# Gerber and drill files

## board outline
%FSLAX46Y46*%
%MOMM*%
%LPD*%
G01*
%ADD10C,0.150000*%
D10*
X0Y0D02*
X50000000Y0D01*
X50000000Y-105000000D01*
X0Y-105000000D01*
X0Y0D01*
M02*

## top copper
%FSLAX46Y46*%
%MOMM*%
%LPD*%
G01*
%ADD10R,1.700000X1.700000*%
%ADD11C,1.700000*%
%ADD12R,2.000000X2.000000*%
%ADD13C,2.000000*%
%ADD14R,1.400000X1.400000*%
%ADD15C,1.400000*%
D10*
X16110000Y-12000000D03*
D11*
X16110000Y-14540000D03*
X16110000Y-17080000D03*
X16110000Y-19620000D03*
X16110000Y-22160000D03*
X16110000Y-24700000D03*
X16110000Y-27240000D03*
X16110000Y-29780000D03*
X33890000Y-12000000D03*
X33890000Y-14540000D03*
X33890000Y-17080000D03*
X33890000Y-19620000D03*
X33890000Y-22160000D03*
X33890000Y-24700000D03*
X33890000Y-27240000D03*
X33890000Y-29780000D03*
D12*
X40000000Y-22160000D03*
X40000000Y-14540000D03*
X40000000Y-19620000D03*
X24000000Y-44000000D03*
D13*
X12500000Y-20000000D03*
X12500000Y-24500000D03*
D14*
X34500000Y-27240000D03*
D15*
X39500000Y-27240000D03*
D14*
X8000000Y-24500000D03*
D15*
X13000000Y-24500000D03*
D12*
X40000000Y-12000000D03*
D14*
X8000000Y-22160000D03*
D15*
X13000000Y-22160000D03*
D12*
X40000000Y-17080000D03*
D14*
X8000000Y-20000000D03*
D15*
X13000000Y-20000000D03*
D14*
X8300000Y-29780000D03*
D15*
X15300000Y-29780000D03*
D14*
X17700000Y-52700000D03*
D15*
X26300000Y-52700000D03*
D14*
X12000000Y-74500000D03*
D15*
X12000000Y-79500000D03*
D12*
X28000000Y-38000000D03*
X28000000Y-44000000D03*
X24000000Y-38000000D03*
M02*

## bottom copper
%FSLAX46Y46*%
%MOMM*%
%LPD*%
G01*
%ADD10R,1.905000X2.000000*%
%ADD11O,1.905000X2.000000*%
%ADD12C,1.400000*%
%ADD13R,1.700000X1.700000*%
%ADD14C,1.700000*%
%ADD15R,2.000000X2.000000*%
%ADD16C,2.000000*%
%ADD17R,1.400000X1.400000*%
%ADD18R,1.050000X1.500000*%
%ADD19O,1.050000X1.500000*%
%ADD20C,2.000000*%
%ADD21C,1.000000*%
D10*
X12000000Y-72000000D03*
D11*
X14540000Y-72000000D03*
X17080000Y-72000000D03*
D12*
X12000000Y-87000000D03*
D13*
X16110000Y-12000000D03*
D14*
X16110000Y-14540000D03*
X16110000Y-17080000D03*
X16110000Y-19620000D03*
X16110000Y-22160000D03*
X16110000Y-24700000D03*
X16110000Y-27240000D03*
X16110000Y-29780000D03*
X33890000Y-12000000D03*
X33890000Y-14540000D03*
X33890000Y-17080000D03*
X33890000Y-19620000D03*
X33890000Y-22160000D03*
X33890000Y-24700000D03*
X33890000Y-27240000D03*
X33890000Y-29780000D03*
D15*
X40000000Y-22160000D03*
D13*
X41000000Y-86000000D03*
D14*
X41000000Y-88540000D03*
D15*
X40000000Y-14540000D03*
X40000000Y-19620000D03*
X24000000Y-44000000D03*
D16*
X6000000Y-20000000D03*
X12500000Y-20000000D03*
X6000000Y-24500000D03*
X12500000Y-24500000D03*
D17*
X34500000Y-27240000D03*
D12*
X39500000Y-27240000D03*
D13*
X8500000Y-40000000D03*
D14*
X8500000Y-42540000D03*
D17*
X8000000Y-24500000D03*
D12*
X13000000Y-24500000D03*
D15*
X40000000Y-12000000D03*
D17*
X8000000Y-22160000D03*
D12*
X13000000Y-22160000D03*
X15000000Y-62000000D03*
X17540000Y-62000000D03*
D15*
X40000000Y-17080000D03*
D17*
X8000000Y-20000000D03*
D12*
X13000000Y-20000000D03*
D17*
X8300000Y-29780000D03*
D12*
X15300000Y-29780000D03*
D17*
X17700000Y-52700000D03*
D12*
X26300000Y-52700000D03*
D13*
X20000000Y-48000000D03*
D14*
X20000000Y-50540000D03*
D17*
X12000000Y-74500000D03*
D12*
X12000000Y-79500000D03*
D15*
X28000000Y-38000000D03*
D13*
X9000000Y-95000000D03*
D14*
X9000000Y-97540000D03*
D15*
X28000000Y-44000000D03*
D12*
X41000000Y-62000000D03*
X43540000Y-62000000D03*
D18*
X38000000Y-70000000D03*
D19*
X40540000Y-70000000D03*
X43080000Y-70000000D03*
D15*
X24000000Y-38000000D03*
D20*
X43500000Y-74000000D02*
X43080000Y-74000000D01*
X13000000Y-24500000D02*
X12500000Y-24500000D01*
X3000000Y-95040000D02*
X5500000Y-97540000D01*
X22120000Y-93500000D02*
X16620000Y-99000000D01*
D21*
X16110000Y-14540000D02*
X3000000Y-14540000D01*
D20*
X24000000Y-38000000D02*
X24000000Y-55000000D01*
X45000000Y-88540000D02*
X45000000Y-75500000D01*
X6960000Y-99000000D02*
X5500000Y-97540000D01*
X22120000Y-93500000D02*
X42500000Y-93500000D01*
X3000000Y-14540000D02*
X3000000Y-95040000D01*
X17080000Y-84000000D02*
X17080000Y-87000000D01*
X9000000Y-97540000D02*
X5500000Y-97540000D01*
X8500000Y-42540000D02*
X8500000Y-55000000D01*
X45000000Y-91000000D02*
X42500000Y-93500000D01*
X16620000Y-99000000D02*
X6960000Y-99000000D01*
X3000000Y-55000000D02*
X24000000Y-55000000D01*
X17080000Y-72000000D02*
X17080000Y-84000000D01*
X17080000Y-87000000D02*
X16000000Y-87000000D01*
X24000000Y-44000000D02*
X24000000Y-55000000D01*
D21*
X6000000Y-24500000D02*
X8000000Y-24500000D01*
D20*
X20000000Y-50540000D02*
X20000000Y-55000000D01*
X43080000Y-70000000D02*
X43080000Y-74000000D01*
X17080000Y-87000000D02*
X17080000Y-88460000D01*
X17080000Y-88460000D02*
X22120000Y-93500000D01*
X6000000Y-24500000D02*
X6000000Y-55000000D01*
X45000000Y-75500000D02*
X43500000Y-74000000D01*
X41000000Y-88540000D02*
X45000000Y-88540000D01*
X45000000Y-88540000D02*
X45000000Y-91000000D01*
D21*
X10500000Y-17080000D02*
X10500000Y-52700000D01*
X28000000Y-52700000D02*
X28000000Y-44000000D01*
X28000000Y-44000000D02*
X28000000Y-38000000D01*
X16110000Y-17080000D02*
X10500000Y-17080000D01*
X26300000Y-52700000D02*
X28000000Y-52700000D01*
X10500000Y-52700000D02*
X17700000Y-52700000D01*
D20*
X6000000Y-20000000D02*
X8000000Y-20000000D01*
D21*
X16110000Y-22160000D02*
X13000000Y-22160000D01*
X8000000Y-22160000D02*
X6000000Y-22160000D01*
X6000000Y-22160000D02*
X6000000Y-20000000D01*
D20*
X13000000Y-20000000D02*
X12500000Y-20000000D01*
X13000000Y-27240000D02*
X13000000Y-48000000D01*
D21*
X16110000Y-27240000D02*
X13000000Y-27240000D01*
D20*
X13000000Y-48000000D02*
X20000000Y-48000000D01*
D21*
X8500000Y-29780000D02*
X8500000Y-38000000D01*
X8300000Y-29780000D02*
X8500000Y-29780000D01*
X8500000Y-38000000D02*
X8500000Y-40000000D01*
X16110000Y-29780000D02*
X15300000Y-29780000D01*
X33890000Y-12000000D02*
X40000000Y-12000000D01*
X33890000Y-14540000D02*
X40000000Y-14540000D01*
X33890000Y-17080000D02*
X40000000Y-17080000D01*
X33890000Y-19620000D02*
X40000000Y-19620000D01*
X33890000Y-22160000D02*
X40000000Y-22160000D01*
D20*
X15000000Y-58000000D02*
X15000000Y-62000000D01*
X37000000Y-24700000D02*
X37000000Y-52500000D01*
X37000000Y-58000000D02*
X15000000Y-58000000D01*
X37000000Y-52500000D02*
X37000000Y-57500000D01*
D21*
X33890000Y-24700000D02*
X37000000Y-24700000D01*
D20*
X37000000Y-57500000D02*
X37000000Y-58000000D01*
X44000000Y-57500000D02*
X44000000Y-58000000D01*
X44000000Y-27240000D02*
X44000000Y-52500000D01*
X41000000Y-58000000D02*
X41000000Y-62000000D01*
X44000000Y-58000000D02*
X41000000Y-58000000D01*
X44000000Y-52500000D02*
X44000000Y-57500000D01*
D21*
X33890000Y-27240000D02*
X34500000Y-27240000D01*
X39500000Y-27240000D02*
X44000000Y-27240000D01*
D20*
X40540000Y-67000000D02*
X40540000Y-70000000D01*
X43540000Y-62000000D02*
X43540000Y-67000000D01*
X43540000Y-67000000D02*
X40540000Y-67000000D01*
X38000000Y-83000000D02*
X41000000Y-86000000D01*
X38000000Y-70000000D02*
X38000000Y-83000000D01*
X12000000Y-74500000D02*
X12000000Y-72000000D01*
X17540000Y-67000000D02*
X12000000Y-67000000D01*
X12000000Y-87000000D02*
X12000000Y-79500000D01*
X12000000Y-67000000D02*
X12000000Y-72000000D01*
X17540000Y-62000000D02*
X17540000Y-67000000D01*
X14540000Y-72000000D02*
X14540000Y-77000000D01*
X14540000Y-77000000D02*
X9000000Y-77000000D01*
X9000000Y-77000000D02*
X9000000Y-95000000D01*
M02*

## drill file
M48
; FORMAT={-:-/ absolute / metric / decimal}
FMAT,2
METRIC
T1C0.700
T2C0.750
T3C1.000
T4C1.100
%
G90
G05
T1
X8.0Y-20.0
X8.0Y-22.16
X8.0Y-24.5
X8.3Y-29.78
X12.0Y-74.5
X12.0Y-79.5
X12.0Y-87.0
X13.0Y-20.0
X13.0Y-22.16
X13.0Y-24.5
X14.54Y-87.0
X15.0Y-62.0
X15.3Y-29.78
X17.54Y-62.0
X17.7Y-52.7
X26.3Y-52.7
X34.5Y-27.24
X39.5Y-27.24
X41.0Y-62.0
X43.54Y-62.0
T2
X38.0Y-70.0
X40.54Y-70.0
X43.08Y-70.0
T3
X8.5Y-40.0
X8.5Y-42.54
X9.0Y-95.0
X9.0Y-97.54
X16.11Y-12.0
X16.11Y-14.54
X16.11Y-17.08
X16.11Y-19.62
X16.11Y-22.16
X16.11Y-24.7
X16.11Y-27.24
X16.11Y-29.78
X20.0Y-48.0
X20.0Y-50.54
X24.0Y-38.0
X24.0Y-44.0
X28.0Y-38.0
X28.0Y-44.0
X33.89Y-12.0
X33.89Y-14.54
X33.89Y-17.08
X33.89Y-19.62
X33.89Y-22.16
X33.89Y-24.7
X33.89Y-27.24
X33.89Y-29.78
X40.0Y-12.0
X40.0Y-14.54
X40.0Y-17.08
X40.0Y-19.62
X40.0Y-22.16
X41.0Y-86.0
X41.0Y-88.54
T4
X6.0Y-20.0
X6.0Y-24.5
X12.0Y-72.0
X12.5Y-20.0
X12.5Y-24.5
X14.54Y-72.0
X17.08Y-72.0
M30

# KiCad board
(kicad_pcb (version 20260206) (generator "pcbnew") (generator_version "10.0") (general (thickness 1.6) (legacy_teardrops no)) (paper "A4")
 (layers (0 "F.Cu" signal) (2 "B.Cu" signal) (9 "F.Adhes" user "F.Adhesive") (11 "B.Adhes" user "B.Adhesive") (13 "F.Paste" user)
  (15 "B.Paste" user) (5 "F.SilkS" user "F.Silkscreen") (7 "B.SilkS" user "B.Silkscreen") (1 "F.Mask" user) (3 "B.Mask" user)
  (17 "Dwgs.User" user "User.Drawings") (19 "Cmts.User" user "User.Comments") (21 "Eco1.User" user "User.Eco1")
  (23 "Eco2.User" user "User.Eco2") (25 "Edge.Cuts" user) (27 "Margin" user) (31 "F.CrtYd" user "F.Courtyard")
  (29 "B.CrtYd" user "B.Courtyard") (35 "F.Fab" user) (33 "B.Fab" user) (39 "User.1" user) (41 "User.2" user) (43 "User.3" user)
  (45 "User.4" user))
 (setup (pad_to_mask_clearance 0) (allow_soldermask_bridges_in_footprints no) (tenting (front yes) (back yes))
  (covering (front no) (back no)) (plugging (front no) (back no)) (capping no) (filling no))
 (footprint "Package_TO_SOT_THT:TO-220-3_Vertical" (layer "F.Cu") (at 12 72)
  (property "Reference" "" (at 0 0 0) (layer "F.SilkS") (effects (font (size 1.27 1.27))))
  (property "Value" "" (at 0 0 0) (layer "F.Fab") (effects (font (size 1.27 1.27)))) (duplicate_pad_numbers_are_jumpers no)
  (pad "1" thru_hole rect (at 0 0) (size 1.905 2) (drill 1.1) (layers "*.Cu" "*.Mask") (remove_unused_layers yes) (keep_end_layers no)
   (zone_layer_connections) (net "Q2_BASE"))
  (pad "2" thru_hole oval (at 2.54 0) (size 1.905 2) (drill 1.1) (layers "*.Cu" "*.Mask") (remove_unused_layers yes) (keep_end_layers no)
   (zone_layer_connections) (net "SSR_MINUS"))
  (pad "3" thru_hole oval (at 5.08 0) (size 1.905 2) (drill 1.1) (layers "*.Cu" "*.Mask") (remove_unused_layers yes) (keep_end_layers no)
   (zone_layer_connections) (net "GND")))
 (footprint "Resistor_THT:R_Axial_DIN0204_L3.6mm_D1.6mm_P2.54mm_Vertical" (layer "F.Cu") (at 12 87)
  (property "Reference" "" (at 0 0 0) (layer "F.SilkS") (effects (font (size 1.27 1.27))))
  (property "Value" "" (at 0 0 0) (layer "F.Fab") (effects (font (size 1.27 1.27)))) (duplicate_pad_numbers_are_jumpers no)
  (pad "1" thru_hole circle (at 0 0) (size 1.4 1.4) (drill 0.7) (layers "*.Cu" "*.Mask") (remove_unused_layers yes) (keep_end_layers no)
   (zone_layer_connections) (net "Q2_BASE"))
  (pad "2" thru_hole circle (at 2.54 0) (size 1.4 1.4) (drill 0.7) (layers "*.Cu" "*.Mask") (remove_unused_layers yes) (keep_end_layers no)
   (zone_layer_connections) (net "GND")))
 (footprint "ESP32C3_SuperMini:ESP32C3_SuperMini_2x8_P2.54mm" (layer "F.Cu") (at 16.11 12)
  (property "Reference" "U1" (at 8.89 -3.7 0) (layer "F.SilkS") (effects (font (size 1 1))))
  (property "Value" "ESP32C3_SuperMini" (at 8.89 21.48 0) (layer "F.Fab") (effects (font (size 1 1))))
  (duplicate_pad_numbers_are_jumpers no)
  (pad "1" thru_hole rect (at 0 0) (size 1.7 1.7) (drill 1) (layers "*.Cu" "*.Mask") (remove_unused_layers no))
  (pad "2" thru_hole circle (at 0 2.54) (size 1.7 1.7) (drill 1) (layers "*.Cu" "*.Mask") (remove_unused_layers no) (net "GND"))
  (pad "3" thru_hole circle (at 0 5.08) (size 1.7 1.7) (drill 1) (layers "*.Cu" "*.Mask") (remove_unused_layers no) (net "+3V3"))
  (pad "4" thru_hole circle (at 0 7.62) (size 1.7 1.7) (drill 1) (layers "*.Cu" "*.Mask") (remove_unused_layers no))
  (pad "5" thru_hole circle (at 0 10.16) (size 1.7 1.7) (drill 1) (layers "*.Cu" "*.Mask") (remove_unused_layers no) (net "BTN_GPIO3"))
  (pad "6" thru_hole circle (at 0 12.7) (size 1.7 1.7) (drill 1) (layers "*.Cu" "*.Mask") (remove_unused_layers no))
  (pad "7" thru_hole circle (at 0 15.24) (size 1.7 1.7) (drill 1) (layers "*.Cu" "*.Mask") (remove_unused_layers no) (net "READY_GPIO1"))
  (pad "8" thru_hole circle (at 0 17.78) (size 1.7 1.7) (drill 1) (layers "*.Cu" "*.Mask") (remove_unused_layers no) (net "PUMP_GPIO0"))
  (pad "9" thru_hole circle (at 17.78 0) (size 1.7 1.7) (drill 1) (layers "*.Cu" "*.Mask") (remove_unused_layers no) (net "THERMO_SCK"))
  (pad "10" thru_hole circle (at 17.78 2.54) (size 1.7 1.7) (drill 1) (layers "*.Cu" "*.Mask") (remove_unused_layers no) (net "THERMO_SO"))
  (pad "11" thru_hole circle (at 17.78 5.08) (size 1.7 1.7) (drill 1) (layers "*.Cu" "*.Mask") (remove_unused_layers no) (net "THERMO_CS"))
  (pad "12" thru_hole circle (at 17.78 7.62) (size 1.7 1.7) (drill 1) (layers "*.Cu" "*.Mask") (remove_unused_layers no) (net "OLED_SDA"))
  (pad "13" thru_hole circle (at 17.78 10.16) (size 1.7 1.7) (drill 1) (layers "*.Cu" "*.Mask") (remove_unused_layers no) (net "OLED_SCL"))
  (pad "14" thru_hole circle (at 17.78 12.7) (size 1.7 1.7) (drill 1) (layers "*.Cu" "*.Mask") (remove_unused_layers no)
   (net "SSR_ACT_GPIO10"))
  (pad "15" thru_hole circle (at 17.78 15.24) (size 1.7 1.7) (drill 1) (layers "*.Cu" "*.Mask") (remove_unused_layers no)
   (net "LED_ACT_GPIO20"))
  (pad "16" thru_hole circle (at 17.78 17.78) (size 1.7 1.7) (drill 1) (layers "*.Cu" "*.Mask") (remove_unused_layers no)))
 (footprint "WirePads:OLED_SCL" (layer "F.Cu") (at 40 22.16)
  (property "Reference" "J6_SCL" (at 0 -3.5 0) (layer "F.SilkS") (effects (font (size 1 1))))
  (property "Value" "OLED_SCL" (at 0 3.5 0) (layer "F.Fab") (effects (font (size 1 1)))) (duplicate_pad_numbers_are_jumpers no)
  (pad "1" thru_hole rect (at 0 0) (size 2 2) (drill 1) (layers "*.Cu" "*.Mask") (remove_unused_layers no) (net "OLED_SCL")))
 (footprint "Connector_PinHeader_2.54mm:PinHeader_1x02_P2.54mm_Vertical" (layer "F.Cu") (at 41 86)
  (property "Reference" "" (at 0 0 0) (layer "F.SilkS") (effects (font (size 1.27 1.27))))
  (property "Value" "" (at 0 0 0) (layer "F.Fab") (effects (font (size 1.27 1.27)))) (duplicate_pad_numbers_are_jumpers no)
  (pad "1" thru_hole rect (at 0 0) (size 1.7 1.7) (drill 1) (layers "*.Cu" "*.Mask") (remove_unused_layers yes) (keep_end_layers no)
   (zone_layer_connections) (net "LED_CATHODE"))
  (pad "2" thru_hole circle (at 0 2.54) (size 1.7 1.7) (drill 1) (layers "*.Cu" "*.Mask") (remove_unused_layers yes) (keep_end_layers no)
   (zone_layer_connections) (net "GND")))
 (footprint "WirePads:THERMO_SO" (layer "F.Cu") (at 40 14.54)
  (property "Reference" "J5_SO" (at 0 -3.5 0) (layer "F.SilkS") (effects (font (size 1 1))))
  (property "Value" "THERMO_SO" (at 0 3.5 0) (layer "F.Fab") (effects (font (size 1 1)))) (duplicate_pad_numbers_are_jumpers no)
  (pad "1" thru_hole rect (at 0 0) (size 2 2) (drill 1) (layers "*.Cu" "*.Mask") (remove_unused_layers no) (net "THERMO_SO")))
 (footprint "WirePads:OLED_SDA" (layer "F.Cu") (at 40 19.62)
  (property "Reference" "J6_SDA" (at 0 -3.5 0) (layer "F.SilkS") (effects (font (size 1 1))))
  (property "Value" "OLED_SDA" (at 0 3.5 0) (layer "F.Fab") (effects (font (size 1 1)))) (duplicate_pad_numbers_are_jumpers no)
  (pad "1" thru_hole rect (at 0 0) (size 2 2) (drill 1) (layers "*.Cu" "*.Mask") (remove_unused_layers no) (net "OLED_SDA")))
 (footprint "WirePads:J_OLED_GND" (layer "F.Cu") (at 24 44)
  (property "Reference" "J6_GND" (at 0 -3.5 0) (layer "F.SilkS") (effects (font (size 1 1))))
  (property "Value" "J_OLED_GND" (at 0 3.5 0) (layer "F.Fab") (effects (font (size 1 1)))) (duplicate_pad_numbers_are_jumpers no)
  (pad "1" thru_hole rect (at 0 0) (size 2 2) (drill 1) (layers "*.Cu" "*.Mask") (remove_unused_layers no) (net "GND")))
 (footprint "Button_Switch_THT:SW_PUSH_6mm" (layer "F.Cu") (at 6 20)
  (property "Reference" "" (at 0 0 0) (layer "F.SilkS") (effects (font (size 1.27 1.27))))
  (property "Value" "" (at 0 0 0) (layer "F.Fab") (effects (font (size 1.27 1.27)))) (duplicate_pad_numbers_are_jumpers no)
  (pad "1" thru_hole circle (at 0 0 90) (size 2 2) (drill 1.1) (layers "*.Cu" "*.Mask") (remove_unused_layers yes) (keep_end_layers no)
   (zone_layer_connections) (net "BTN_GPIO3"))
  (pad "1" thru_hole circle (at 6.5 0 90) (size 2 2) (drill 1.1) (layers "*.Cu" "*.Mask") (remove_unused_layers yes) (keep_end_layers no)
   (zone_layer_connections) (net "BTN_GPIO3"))
  (pad "2" thru_hole circle (at 0 4.5 90) (size 2 2) (drill 1.1) (layers "*.Cu" "*.Mask") (remove_unused_layers yes) (keep_end_layers no)
   (zone_layer_connections) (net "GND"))
  (pad "2" thru_hole circle (at 6.5 4.5 90) (size 2 2) (drill 1.1) (layers "*.Cu" "*.Mask") (remove_unused_layers yes) (keep_end_layers no)
   (zone_layer_connections) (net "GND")))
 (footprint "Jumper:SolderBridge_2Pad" (layer "F.Cu") (at 34.5 27.24)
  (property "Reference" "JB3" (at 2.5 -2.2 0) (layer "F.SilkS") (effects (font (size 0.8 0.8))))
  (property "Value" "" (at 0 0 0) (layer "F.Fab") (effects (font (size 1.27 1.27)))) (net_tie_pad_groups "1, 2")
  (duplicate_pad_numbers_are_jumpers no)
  (pad "1" thru_hole rect (at 0 0) (size 1.4 1.4) (drill 0.7) (layers "*.Cu" "*.Mask") (remove_unused_layers no) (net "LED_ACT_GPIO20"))
  (pad "2" thru_hole circle (at 5 0) (size 1.4 1.4) (drill 0.7) (layers "*.Cu" "*.Mask") (remove_unused_layers no) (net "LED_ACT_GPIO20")))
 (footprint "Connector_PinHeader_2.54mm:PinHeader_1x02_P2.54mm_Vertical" (layer "F.Cu") (at 8.5 40)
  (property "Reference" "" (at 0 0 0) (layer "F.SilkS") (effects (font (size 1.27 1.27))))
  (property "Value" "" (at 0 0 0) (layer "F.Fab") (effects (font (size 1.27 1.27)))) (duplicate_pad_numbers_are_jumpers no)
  (pad "1" thru_hole rect (at 0 0) (size 1.7 1.7) (drill 1) (layers "*.Cu" "*.Mask") (remove_unused_layers yes) (keep_end_layers no)
   (zone_layer_connections) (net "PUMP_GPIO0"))
  (pad "2" thru_hole circle (at 0 2.54) (size 1.7 1.7) (drill 1) (layers "*.Cu" "*.Mask") (remove_unused_layers yes) (keep_end_layers no)
   (zone_layer_connections) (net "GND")))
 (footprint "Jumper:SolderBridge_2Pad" (layer "F.Cu") (at 8 24.5)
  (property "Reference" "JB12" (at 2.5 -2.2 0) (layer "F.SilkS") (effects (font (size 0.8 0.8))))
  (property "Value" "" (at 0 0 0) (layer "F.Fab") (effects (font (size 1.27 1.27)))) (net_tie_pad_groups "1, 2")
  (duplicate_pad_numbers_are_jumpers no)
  (pad "1" thru_hole rect (at 0 0) (size 1.4 1.4) (drill 0.7) (layers "*.Cu" "*.Mask") (remove_unused_layers no) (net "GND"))
  (pad "2" thru_hole circle (at 5 0) (size 1.4 1.4) (drill 0.7) (layers "*.Cu" "*.Mask") (remove_unused_layers no) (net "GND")))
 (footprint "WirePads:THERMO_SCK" (layer "F.Cu") (at 40 12)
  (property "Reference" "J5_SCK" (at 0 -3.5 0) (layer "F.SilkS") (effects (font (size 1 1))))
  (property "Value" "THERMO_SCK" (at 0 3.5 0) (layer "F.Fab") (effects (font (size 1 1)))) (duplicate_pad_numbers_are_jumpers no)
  (pad "1" thru_hole rect (at 0 0) (size 2 2) (drill 1) (layers "*.Cu" "*.Mask") (remove_unused_layers no) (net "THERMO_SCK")))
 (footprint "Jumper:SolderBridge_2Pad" (layer "F.Cu") (at 8 22.16)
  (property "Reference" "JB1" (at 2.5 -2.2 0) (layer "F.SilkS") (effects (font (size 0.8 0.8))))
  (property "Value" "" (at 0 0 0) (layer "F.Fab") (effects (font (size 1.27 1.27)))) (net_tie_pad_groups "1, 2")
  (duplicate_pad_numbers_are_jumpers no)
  (pad "1" thru_hole rect (at 0 0) (size 1.4 1.4) (drill 0.7) (layers "*.Cu" "*.Mask") (remove_unused_layers no) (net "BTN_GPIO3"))
  (pad "2" thru_hole circle (at 5 0) (size 1.4 1.4) (drill 0.7) (layers "*.Cu" "*.Mask") (remove_unused_layers no) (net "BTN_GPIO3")))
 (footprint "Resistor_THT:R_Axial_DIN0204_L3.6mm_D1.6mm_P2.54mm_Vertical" (layer "F.Cu") (at 15 62)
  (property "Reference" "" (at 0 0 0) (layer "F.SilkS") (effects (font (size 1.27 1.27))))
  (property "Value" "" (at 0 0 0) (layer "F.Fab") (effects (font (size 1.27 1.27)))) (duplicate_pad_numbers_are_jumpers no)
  (pad "1" thru_hole circle (at 0 0) (size 1.4 1.4) (drill 0.7) (layers "*.Cu" "*.Mask") (remove_unused_layers yes) (keep_end_layers no)
   (zone_layer_connections) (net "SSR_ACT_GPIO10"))
  (pad "2" thru_hole circle (at 2.54 0) (size 1.4 1.4) (drill 0.7) (layers "*.Cu" "*.Mask") (remove_unused_layers yes) (keep_end_layers no)
   (zone_layer_connections) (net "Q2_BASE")))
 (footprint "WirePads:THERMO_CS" (layer "F.Cu") (at 40 17.08)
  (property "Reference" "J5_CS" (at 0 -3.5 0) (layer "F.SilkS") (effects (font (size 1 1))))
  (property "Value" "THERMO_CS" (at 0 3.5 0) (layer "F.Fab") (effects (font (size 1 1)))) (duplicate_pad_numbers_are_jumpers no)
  (pad "1" thru_hole rect (at 0 0) (size 2 2) (drill 1) (layers "*.Cu" "*.Mask") (remove_unused_layers no) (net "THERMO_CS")))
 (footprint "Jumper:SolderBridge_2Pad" (layer "F.Cu") (at 8 20)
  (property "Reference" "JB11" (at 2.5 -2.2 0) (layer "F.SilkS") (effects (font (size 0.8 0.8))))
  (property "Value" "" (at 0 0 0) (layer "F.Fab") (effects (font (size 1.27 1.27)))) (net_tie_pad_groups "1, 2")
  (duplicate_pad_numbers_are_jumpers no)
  (pad "1" thru_hole rect (at 0 0) (size 1.4 1.4) (drill 0.7) (layers "*.Cu" "*.Mask") (remove_unused_layers no) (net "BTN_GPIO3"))
  (pad "2" thru_hole circle (at 5 0) (size 1.4 1.4) (drill 0.7) (layers "*.Cu" "*.Mask") (remove_unused_layers no) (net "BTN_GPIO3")))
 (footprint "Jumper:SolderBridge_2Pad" (layer "F.Cu") (at 8.3 29.78)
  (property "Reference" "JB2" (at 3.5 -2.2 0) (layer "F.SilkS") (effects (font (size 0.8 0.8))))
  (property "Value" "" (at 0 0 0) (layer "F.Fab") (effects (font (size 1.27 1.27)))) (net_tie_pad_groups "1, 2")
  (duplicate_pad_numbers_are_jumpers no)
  (pad "1" thru_hole rect (at 0 0) (size 1.4 1.4) (drill 0.7) (layers "*.Cu" "*.Mask") (remove_unused_layers no) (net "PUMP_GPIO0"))
  (pad "2" thru_hole circle (at 7 0) (size 1.4 1.4) (drill 0.7) (layers "*.Cu" "*.Mask") (remove_unused_layers no) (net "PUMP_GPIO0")))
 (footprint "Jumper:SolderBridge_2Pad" (layer "F.Cu") (at 17.7 52.7)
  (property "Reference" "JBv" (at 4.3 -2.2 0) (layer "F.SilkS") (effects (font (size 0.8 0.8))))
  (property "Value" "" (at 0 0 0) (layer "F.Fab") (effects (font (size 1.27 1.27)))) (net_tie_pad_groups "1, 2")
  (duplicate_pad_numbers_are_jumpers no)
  (pad "1" thru_hole rect (at 0 0) (size 1.4 1.4) (drill 0.7) (layers "*.Cu" "*.Mask") (remove_unused_layers no) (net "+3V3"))
  (pad "2" thru_hole circle (at 8.6 0) (size 1.4 1.4) (drill 0.7) (layers "*.Cu" "*.Mask") (remove_unused_layers no) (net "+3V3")))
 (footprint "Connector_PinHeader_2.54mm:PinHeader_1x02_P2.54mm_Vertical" (layer "F.Cu") (at 20 48)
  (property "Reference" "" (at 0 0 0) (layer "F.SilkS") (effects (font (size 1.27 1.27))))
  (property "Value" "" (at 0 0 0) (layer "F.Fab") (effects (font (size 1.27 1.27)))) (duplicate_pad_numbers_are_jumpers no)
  (pad "1" thru_hole rect (at 0 0) (size 1.7 1.7) (drill 1) (layers "*.Cu" "*.Mask") (remove_unused_layers yes) (keep_end_layers no)
   (zone_layer_connections) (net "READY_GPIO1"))
  (pad "2" thru_hole circle (at 0 2.54) (size 1.7 1.7) (drill 1) (layers "*.Cu" "*.Mask") (remove_unused_layers yes) (keep_end_layers no)
   (zone_layer_connections) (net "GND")))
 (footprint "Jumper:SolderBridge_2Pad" (layer "F.Cu") (at 12 74.5)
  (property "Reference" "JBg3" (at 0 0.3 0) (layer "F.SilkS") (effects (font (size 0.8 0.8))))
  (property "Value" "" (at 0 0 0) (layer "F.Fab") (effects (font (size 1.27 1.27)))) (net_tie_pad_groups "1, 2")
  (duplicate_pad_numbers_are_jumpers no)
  (pad "1" thru_hole rect (at 0 0) (size 1.4 1.4) (drill 0.7) (layers "*.Cu" "*.Mask") (remove_unused_layers no) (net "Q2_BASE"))
  (pad "2" thru_hole circle (at 0 5) (size 1.4 1.4) (drill 0.7) (layers "*.Cu" "*.Mask") (remove_unused_layers no) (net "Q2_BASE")))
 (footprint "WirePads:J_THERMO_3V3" (layer "F.Cu") (at 28 38)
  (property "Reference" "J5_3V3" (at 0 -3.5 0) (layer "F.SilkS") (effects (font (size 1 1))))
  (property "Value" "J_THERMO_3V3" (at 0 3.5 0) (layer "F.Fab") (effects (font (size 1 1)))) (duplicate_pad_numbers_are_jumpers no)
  (pad "1" thru_hole rect (at 0 0) (size 2 2) (drill 1) (layers "*.Cu" "*.Mask") (remove_unused_layers no) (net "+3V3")))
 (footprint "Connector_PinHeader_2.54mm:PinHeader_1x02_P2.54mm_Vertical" (layer "F.Cu") (at 9 95)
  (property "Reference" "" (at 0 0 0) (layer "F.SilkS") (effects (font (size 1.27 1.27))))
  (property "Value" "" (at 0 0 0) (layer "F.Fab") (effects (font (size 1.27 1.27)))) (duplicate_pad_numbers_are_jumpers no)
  (pad "1" thru_hole rect (at 0 0) (size 1.7 1.7) (drill 1) (layers "*.Cu" "*.Mask") (remove_unused_layers yes) (keep_end_layers no)
   (zone_layer_connections) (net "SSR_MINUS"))
  (pad "2" thru_hole circle (at 0 2.54) (size 1.7 1.7) (drill 1) (layers "*.Cu" "*.Mask") (remove_unused_layers yes) (keep_end_layers no)
   (zone_layer_connections) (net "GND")))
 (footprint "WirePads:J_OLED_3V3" (layer "F.Cu") (at 28 44)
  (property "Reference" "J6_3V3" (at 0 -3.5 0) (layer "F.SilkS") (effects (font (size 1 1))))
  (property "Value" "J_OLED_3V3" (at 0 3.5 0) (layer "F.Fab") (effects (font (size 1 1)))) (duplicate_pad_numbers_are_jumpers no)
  (pad "1" thru_hole rect (at 0 0) (size 2 2) (drill 1) (layers "*.Cu" "*.Mask") (remove_unused_layers no) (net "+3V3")))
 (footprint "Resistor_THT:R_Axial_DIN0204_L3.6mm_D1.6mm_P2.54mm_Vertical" (layer "F.Cu") (at 41 62)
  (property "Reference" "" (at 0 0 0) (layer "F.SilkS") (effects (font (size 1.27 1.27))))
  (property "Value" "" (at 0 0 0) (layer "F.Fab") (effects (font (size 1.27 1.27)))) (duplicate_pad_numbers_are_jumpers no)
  (pad "1" thru_hole circle (at 0 0) (size 1.4 1.4) (drill 0.7) (layers "*.Cu" "*.Mask") (remove_unused_layers yes) (keep_end_layers no)
   (zone_layer_connections) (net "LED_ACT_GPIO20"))
  (pad "2" thru_hole circle (at 2.54 0) (size 1.4 1.4) (drill 0.7) (layers "*.Cu" "*.Mask") (remove_unused_layers yes) (keep_end_layers no)
   (zone_layer_connections) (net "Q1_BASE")))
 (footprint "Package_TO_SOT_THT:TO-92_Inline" (layer "F.Cu") (at 38 70)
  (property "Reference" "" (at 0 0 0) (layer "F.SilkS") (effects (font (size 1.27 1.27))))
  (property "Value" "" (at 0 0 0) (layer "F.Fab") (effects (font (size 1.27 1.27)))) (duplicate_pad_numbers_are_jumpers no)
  (pad "1" thru_hole rect (at 0 0) (size 1.05 1.5) (drill 0.75) (layers "*.Cu" "*.Mask") (remove_unused_layers yes) (keep_end_layers no)
   (zone_layer_connections) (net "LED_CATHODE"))
  (pad "2" thru_hole oval (at 2.54 0) (size 1.05 1.5) (drill 0.75) (layers "*.Cu" "*.Mask") (remove_unused_layers yes) (keep_end_layers no)
   (zone_layer_connections) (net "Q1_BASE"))
  (pad "3" thru_hole oval (at 5.08 0) (size 1.05 1.5) (drill 0.75) (layers "*.Cu" "*.Mask") (remove_unused_layers yes) (keep_end_layers no)
   (zone_layer_connections) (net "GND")))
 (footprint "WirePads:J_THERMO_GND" (layer "F.Cu") (at 24 38)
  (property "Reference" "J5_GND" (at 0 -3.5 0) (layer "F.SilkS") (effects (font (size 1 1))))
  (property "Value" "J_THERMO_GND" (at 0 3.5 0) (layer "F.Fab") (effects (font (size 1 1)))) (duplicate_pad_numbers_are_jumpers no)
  (pad "1" thru_hole rect (at 0 0) (size 2 2) (drill 1) (layers "*.Cu" "*.Mask") (remove_unused_layers no) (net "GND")))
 (gr_rect (start 0 0) (end 50 105) (stroke (width 0.15) (type solid)) (fill no) (layer "Edge.Cuts"))
 (segment (start 43.5 74) (end 43.08 74) (width 2) (layer "B.Cu") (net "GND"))
 (segment (start 13 24.5) (end 12.5 24.5) (width 2) (layer "B.Cu") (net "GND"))
 (segment (start 3 95.04) (end 5.5 97.54) (width 2) (layer "B.Cu") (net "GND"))
 (segment (start 22.12 93.5) (end 16.62 99) (width 2) (layer "B.Cu") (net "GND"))
 (segment (start 16.11 14.54) (end 3 14.54) (width 1) (layer "B.Cu") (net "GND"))
 (segment (start 24 38) (end 24 55) (width 2) (layer "B.Cu") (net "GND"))
 (segment (start 45 88.54) (end 45 75.5) (width 2) (layer "B.Cu") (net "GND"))
 (segment (start 6.96 99) (end 5.5 97.54) (width 2) (layer "B.Cu") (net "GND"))
 (segment (start 22.12 93.5) (end 42.5 93.5) (width 2) (layer "B.Cu") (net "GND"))
 (segment (start 3 14.54) (end 3 95.04) (width 2) (layer "B.Cu") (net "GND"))
 (segment (start 17.08 84) (end 17.08 87) (width 2) (layer "B.Cu") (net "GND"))
 (segment (start 9 97.54) (end 5.5 97.54) (width 2) (layer "B.Cu") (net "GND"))
 (segment (start 8.5 42.54) (end 8.5 55) (width 2) (layer "B.Cu") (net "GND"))
 (segment (start 45 91) (end 42.5 93.5) (width 2) (layer "B.Cu") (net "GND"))
 (segment (start 16.62 99) (end 6.96 99) (width 2) (layer "B.Cu") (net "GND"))
 (segment (start 3 55) (end 24 55) (width 2) (layer "B.Cu") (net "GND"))
 (segment (start 17.08 72) (end 17.08 84) (width 2) (layer "B.Cu") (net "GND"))
 (segment (start 17.08 87) (end 16 87) (width 2) (layer "B.Cu") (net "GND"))
 (segment (start 24 44) (end 24 55) (width 2) (layer "B.Cu") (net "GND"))
 (segment (start 6 24.5) (end 8 24.5) (width 1) (layer "B.Cu") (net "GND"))
 (segment (start 20 50.54) (end 20 55) (width 2) (layer "B.Cu") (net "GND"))
 (segment (start 43.08 70) (end 43.08 74) (width 2) (layer "B.Cu") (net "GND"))
 (segment (start 17.08 87) (end 17.08 88.46) (width 2) (layer "B.Cu") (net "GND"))
 (segment (start 17.08 88.46) (end 22.12 93.5) (width 2) (layer "B.Cu") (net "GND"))
 (segment (start 6 24.5) (end 6 55) (width 2) (layer "B.Cu") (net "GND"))
 (segment (start 45 75.5) (end 43.5 74) (width 2) (layer "B.Cu") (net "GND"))
 (segment (start 41 88.54) (end 45 88.54) (width 2) (layer "B.Cu") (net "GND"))
 (segment (start 45 88.54) (end 45 91) (width 2) (layer "B.Cu") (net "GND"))
 (segment (start 10.5 17.08) (end 10.5 52.7) (width 1) (layer "B.Cu") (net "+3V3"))
 (segment (start 28 52.7) (end 28 44) (width 1) (layer "B.Cu") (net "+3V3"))
 (segment (start 28 44) (end 28 38) (width 1) (layer "B.Cu") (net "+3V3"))
 (segment (start 16.11 17.08) (end 10.5 17.08) (width 1) (layer "B.Cu") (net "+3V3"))
 (segment (start 26.3 52.7) (end 28 52.7) (width 1) (layer "B.Cu") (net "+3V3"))
 (segment (start 10.5 52.7) (end 17.7 52.7) (width 1) (layer "B.Cu") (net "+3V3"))
 (segment (start 6 20) (end 8 20) (width 2) (layer "B.Cu") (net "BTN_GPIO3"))
 (segment (start 16.11 22.16) (end 13 22.16) (width 1) (layer "B.Cu") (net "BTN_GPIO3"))
 (segment (start 8 22.16) (end 6 22.16) (width 1) (layer "B.Cu") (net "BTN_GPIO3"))
 (segment (start 6 22.16) (end 6 20) (width 1) (layer "B.Cu") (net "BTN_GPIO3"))
 (segment (start 13 20) (end 12.5 20) (width 2) (layer "B.Cu") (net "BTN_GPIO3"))
 (segment (start 13 27.24) (end 13 48) (width 2) (layer "B.Cu") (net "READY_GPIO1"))
 (segment (start 16.11 27.24) (end 13 27.24) (width 1) (layer "B.Cu") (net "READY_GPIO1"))
 (segment (start 13 48) (end 20 48) (width 2) (layer "B.Cu") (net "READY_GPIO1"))
 (segment (start 8.5 29.78) (end 8.5 38) (width 1) (layer "B.Cu") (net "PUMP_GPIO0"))
 (segment (start 8.3 29.78) (end 8.5 29.78) (width 1) (layer "B.Cu") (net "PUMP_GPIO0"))
 (segment (start 8.5 38) (end 8.5 40) (width 1) (layer "B.Cu") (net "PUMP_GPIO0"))
 (segment (start 16.11 29.78) (end 15.3 29.78) (width 1) (layer "B.Cu") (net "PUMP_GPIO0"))
 (segment (start 33.89 12) (end 40 12) (width 1) (layer "B.Cu") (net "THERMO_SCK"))
 (segment (start 33.89 14.54) (end 40 14.54) (width 1) (layer "B.Cu") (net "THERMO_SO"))
 (segment (start 33.89 17.08) (end 40 17.08) (width 1) (layer "B.Cu") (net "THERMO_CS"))
 (segment (start 33.89 19.62) (end 40 19.62) (width 1) (layer "B.Cu") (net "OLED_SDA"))
 (segment (start 33.89 22.16) (end 40 22.16) (width 1) (layer "B.Cu") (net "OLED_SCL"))
 (segment (start 15 58) (end 15 62) (width 2) (layer "B.Cu") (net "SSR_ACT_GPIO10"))
 (segment (start 37 24.7) (end 37 52.5) (width 2) (layer "B.Cu") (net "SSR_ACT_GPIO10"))
 (segment (start 37 58) (end 15 58) (width 2) (layer "B.Cu") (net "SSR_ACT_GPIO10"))
 (segment (start 37 52.5) (end 37 57.5) (width 2) (layer "B.Cu") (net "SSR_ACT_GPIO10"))
 (segment (start 33.89 24.7) (end 37 24.7) (width 1) (layer "B.Cu") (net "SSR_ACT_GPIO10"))
 (segment (start 37 57.5) (end 37 58) (width 2) (layer "B.Cu") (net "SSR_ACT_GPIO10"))
 (segment (start 44 57.5) (end 44 58) (width 2) (layer "B.Cu") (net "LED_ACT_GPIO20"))
 (segment (start 44 27.24) (end 44 52.5) (width 2) (layer "B.Cu") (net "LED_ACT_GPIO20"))
 (segment (start 41 58) (end 41 62) (width 2) (layer "B.Cu") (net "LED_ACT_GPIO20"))
 (segment (start 44 58) (end 41 58) (width 2) (layer "B.Cu") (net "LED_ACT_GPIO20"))
 (segment (start 44 52.5) (end 44 57.5) (width 2) (layer "B.Cu") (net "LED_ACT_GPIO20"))
 (segment (start 33.89 27.24) (end 34.5 27.24) (width 1) (layer "B.Cu") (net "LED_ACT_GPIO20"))
 (segment (start 39.5 27.24) (end 44 27.24) (width 1) (layer "B.Cu") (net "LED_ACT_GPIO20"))
 (segment (start 40.54 67) (end 40.54 70) (width 2) (layer "B.Cu") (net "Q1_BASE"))
 (segment (start 43.54 62) (end 43.54 67) (width 2) (layer "B.Cu") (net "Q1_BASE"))
 (segment (start 43.54 67) (end 40.54 67) (width 2) (layer "B.Cu") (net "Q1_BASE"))
 (segment (start 38 83) (end 41 86) (width 2) (layer "B.Cu") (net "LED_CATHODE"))
 (segment (start 38 70) (end 38 83) (width 2) (layer "B.Cu") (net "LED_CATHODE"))
 (segment (start 12 74.5) (end 12 72) (width 2) (layer "B.Cu") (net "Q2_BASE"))
 (segment (start 17.54 67) (end 12 67) (width 2) (layer "B.Cu") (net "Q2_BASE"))
 (segment (start 12 87) (end 12 79.5) (width 2) (layer "B.Cu") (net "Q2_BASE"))
 (segment (start 12 67) (end 12 72) (width 2) (layer "B.Cu") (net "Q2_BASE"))
 (segment (start 17.54 62) (end 17.54 67) (width 2) (layer "B.Cu") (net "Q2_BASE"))
 (segment (start 14.54 72) (end 14.54 77) (width 2) (layer "B.Cu") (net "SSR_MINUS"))
 (segment (start 14.54 77) (end 9 77) (width 2) (layer "B.Cu") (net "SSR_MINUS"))
 (segment (start 9 77) (end 9 95) (width 2) (layer "B.Cu") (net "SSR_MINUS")))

